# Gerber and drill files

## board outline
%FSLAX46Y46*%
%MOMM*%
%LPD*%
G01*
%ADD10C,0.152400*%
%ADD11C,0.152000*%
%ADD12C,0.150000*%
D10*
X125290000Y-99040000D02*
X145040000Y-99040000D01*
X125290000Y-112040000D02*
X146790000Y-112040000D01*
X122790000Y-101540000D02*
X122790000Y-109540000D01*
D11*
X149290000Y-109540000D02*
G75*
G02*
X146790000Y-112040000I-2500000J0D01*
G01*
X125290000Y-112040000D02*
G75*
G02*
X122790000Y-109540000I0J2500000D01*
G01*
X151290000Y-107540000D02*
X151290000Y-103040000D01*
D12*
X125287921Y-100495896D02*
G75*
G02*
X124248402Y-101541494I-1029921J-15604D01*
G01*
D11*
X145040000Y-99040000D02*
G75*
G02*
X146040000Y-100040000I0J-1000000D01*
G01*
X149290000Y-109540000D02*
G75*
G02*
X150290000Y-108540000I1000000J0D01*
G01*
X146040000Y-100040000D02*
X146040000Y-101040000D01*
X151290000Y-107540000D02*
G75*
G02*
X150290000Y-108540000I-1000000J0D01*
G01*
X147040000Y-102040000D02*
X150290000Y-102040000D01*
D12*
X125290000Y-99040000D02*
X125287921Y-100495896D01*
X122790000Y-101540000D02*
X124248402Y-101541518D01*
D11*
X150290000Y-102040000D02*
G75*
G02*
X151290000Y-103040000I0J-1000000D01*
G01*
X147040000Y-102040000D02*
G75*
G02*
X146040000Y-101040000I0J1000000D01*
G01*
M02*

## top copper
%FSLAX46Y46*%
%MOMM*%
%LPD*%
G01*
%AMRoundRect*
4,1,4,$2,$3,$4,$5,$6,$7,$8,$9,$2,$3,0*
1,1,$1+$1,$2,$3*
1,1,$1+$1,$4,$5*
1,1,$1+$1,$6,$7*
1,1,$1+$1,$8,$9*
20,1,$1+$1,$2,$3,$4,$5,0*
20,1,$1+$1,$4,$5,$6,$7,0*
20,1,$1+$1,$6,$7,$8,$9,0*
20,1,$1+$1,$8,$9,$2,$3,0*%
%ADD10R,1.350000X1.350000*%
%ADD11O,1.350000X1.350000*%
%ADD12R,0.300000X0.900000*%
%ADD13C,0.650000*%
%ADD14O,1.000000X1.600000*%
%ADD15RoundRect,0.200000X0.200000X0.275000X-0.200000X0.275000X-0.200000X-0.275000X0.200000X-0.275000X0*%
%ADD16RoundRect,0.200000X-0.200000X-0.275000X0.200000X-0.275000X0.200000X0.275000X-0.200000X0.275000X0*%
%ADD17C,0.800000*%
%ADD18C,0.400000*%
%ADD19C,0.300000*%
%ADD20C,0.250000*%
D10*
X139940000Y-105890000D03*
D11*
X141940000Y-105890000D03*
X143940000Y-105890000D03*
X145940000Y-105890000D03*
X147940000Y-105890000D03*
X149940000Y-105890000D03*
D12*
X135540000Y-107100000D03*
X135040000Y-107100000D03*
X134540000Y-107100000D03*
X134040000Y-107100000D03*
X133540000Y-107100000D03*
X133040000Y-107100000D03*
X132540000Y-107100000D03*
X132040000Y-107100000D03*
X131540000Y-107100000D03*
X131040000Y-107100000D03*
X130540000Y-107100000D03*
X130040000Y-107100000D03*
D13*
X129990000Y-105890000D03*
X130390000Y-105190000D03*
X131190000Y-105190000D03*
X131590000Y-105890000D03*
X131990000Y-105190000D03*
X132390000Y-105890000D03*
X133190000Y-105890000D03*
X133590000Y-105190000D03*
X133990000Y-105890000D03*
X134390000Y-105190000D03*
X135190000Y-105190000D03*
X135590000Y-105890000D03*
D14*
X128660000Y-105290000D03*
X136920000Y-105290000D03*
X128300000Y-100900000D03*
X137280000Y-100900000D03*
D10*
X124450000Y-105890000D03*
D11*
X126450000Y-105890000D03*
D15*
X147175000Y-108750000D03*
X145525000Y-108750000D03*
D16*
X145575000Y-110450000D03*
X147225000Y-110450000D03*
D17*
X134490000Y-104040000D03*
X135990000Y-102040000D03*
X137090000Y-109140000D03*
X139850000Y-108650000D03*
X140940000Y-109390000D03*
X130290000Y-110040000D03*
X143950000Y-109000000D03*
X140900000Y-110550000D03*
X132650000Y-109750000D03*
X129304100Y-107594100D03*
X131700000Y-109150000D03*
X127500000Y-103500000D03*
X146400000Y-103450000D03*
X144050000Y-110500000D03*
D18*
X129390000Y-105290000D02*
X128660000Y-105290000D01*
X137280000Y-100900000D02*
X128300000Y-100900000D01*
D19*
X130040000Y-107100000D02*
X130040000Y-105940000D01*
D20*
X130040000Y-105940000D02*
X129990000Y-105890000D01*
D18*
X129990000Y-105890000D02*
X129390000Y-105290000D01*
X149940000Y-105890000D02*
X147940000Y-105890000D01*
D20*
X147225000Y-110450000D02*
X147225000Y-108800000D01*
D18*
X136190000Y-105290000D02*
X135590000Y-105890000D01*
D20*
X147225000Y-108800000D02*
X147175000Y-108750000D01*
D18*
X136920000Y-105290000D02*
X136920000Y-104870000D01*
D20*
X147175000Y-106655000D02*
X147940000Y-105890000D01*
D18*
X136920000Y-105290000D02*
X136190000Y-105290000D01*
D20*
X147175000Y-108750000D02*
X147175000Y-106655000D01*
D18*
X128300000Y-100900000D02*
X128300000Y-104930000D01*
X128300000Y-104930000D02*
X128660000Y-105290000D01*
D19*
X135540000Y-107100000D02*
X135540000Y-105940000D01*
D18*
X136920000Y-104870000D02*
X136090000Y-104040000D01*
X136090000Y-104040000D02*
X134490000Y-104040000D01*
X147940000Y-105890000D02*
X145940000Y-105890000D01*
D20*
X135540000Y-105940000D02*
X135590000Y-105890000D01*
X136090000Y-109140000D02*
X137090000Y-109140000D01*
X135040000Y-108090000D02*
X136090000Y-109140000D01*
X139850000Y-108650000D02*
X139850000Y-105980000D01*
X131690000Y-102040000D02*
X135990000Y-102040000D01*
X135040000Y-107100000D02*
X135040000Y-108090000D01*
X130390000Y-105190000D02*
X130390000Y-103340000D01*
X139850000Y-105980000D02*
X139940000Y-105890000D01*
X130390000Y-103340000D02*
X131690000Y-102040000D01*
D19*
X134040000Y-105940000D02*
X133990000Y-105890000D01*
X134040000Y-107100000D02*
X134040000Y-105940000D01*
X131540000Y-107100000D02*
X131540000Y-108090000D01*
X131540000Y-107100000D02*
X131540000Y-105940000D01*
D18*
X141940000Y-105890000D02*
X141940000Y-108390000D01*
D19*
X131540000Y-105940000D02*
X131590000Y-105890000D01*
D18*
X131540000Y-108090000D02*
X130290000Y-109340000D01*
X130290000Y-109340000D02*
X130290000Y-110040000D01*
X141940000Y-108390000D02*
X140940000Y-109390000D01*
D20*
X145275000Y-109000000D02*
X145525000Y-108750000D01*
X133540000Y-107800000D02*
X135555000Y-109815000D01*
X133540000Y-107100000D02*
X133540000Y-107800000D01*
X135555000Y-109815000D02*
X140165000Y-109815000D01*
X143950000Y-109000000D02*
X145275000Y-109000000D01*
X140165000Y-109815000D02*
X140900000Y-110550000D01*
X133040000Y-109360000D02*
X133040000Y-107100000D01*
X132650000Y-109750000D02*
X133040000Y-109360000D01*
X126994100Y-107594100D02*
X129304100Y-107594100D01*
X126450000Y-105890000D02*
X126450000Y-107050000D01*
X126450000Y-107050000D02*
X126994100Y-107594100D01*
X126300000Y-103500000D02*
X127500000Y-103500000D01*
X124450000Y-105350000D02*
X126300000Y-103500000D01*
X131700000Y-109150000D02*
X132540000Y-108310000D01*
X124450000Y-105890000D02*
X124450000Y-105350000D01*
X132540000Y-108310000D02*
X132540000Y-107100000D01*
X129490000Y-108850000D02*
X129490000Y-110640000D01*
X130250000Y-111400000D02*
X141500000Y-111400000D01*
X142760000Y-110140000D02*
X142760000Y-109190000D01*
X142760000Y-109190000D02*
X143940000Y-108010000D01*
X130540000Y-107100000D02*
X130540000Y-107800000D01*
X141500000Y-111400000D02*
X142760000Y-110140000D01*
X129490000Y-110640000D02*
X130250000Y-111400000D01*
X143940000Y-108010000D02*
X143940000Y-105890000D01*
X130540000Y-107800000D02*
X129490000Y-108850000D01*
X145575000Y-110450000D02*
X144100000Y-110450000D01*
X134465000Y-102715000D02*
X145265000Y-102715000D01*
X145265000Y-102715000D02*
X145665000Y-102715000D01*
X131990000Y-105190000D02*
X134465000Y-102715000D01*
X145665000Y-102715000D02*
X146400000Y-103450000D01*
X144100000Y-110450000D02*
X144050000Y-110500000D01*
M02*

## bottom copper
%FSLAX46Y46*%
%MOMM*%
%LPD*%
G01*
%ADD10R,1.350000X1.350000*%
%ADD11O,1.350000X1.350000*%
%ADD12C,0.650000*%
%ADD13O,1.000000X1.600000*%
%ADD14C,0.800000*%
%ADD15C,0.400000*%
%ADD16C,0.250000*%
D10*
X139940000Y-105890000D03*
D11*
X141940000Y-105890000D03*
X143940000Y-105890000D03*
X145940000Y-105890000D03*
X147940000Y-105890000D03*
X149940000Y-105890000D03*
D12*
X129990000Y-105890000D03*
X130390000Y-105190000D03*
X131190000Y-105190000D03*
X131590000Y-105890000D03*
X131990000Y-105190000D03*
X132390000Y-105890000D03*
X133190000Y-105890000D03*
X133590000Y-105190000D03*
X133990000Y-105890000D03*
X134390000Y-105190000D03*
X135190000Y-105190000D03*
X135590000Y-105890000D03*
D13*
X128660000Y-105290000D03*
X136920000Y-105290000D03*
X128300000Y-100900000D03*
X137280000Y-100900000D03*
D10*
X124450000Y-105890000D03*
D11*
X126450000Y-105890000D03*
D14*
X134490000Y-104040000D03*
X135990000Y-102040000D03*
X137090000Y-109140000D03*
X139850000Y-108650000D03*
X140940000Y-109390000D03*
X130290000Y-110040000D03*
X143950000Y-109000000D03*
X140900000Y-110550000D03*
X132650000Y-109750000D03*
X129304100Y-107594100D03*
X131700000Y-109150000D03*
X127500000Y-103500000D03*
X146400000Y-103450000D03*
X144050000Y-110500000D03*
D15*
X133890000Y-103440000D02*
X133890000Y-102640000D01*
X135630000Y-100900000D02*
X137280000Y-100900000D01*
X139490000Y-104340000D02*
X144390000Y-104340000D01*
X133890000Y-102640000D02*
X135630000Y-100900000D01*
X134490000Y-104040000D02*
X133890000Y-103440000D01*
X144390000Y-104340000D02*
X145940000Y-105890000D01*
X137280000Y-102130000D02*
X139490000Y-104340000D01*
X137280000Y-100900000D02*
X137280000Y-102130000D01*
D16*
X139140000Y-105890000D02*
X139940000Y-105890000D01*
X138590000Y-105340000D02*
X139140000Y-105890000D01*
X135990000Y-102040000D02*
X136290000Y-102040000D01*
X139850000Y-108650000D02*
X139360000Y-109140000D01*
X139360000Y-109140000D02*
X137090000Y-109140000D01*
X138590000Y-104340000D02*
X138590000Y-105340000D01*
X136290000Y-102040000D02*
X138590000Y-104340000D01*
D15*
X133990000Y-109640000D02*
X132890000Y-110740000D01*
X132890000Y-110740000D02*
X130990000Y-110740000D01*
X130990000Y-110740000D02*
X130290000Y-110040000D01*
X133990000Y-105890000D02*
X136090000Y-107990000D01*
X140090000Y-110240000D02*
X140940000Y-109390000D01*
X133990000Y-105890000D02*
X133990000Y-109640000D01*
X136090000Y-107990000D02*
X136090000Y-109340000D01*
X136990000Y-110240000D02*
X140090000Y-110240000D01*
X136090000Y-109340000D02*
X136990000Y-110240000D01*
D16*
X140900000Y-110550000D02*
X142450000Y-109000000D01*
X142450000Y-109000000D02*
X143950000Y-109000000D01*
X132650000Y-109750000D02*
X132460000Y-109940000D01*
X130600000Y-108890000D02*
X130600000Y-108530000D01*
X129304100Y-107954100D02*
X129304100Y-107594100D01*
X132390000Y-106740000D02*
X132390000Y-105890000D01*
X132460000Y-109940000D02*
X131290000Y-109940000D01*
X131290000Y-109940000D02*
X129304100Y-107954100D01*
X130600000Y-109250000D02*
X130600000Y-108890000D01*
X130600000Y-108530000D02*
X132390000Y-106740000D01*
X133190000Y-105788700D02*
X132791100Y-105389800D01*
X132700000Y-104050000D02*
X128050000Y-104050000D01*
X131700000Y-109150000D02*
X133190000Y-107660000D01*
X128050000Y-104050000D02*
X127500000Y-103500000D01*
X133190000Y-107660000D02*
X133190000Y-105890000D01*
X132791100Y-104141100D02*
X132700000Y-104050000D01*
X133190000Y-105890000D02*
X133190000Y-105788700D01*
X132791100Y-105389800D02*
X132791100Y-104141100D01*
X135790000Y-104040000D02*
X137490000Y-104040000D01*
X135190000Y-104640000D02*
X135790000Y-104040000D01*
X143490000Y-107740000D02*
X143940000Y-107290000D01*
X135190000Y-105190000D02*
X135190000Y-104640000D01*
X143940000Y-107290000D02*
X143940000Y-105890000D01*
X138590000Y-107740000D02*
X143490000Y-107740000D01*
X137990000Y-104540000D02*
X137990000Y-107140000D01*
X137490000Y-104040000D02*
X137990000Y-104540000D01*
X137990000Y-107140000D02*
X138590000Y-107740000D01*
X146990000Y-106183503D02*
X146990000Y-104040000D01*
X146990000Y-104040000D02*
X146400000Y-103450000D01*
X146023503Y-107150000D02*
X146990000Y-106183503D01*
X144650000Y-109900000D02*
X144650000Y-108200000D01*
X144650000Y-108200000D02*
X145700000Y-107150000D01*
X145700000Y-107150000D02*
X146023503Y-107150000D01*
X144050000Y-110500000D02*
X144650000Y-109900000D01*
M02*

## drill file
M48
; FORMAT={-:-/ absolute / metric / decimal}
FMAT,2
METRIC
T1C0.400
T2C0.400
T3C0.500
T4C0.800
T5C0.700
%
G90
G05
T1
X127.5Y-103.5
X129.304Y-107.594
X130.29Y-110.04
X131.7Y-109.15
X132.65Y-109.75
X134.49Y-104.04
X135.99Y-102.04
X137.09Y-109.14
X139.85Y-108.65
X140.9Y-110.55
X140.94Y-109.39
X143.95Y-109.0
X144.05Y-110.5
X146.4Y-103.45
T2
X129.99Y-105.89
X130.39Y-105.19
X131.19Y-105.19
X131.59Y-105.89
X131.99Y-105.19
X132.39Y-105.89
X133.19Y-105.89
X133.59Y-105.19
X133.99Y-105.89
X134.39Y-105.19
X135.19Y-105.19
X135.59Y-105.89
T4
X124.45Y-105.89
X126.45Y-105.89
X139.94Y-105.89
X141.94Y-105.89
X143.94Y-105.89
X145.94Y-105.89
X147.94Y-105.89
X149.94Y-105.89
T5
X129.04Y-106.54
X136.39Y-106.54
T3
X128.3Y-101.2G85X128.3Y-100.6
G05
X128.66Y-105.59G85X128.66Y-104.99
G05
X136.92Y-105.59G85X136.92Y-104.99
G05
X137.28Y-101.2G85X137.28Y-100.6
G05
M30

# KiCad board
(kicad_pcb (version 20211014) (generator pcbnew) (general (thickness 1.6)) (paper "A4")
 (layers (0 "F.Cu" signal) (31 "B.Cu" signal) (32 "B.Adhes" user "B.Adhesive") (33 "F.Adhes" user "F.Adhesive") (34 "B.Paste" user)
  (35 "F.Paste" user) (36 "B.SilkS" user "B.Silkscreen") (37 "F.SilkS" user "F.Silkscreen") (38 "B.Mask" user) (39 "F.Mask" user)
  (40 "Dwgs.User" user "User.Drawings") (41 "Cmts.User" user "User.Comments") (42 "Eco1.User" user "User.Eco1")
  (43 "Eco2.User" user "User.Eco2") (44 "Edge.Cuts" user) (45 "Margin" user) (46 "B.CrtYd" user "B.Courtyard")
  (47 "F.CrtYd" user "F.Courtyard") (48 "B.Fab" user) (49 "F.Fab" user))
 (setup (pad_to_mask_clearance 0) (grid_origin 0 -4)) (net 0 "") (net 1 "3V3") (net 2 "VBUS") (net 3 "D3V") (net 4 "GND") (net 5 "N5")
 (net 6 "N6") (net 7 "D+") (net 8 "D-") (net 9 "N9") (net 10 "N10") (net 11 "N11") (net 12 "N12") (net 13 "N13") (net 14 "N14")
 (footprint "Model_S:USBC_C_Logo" (layer "F.Cu") (at 130.3 110)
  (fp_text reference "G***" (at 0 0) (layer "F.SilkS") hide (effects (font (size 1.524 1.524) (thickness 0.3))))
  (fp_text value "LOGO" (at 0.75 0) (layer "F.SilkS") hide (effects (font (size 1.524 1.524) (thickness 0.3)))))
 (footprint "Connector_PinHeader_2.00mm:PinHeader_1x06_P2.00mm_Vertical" (layer "F.Cu") (at 139.94 105.89 90)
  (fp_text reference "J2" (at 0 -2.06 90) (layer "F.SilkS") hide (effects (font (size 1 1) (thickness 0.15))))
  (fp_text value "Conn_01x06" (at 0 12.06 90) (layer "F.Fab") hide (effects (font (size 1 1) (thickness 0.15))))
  (pad "1" thru_hole rect locked (at 0 0 90) (size 1.35 1.35) (drill 0.8) (layers *.Cu *.Mask) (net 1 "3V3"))
  (pad "2" thru_hole oval locked (at 0 2 90) (size 1.35 1.35) (drill 0.8) (layers *.Cu *.Mask) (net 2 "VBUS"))
  (pad "3" thru_hole oval locked (at 0 4 90) (size 1.35 1.35) (drill 0.8) (layers *.Cu *.Mask) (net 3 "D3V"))
  (pad "4" thru_hole oval locked (at 0 6 90) (size 1.35 1.35) (drill 0.8) (layers *.Cu *.Mask) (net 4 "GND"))
  (pad "5" thru_hole oval locked (at 0 8 90) (size 1.35 1.35) (drill 0.8) (layers *.Cu *.Mask) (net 4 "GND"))
  (pad "6" thru_hole oval locked (at 0 10 90) (size 1.35 1.35) (drill 0.8) (layers *.Cu *.Mask) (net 4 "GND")))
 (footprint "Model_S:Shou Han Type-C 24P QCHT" (layer "F.Cu") (at 132.79 99.04 180)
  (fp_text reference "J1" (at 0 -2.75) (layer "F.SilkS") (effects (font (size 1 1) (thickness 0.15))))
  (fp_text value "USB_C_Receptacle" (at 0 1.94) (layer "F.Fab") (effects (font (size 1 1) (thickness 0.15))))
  (pad "" np_thru_hole circle locked (at 3.75 -7.5 180) (size 0.7 0.7) (drill 0.7) (layers *.Cu *.Mask))
  (pad "" np_thru_hole circle locked (at -3.6 -7.5 180) (size 0.7 0.7) (drill 0.7) (layers *.Cu *.Mask))
  (pad "A1" smd rect locked (at -2.75 -8.06 180) (size 0.3 0.9) (layers "F.Cu" "F.Paste" "F.Mask") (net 4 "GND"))
  (pad "A2" smd rect locked (at -2.25 -8.06 180) (size 0.3 0.9) (layers "F.Cu" "F.Paste" "F.Mask") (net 1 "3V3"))
  (pad "A3" smd rect locked (at -1.75 -8.06 180) (size 0.3 0.9) (layers "F.Cu" "F.Paste" "F.Mask") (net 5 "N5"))
  (pad "A4" smd rect locked (at -1.25 -8.06 180) (size 0.3 0.9) (layers "F.Cu" "F.Paste" "F.Mask") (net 2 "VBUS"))
  (pad "A5" smd rect locked (at -0.75 -8.06 180) (size 0.3 0.9) (layers "F.Cu" "F.Paste" "F.Mask") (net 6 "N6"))
  (pad "A6" smd rect locked (at -0.25 -8.06 180) (size 0.3 0.9) (layers "F.Cu" "F.Paste" "F.Mask") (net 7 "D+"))
  (pad "A7" smd rect locked (at 0.25 -8.06 180) (size 0.3 0.9) (layers "F.Cu" "F.Paste" "F.Mask") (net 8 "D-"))
  (pad "A8" smd rect locked (at 0.75 -8.06 180) (size 0.3 0.9) (layers "F.Cu" "F.Paste" "F.Mask") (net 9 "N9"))
  (pad "A9" smd rect locked (at 1.25 -8.06 180) (size 0.3 0.9) (layers "F.Cu" "F.Paste" "F.Mask") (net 2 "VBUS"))
  (pad "A10" smd rect locked (at 1.75 -8.06 180) (size 0.3 0.9) (layers "F.Cu" "F.Paste" "F.Mask") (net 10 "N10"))
  (pad "A11" smd rect locked (at 2.25 -8.06 180) (size 0.3 0.9) (layers "F.Cu" "F.Paste" "F.Mask") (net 3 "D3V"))
  (pad "A12" smd rect locked (at 2.75 -8.06 180) (size 0.3 0.9) (layers "F.Cu" "F.Paste" "F.Mask") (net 4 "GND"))
  (pad "B1" thru_hole circle locked (at 2.8 -6.85 180) (size 0.65 0.65) (drill 0.4) (layers *.Cu *.Mask) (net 4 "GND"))
  (pad "B2" thru_hole circle locked (at 2.4 -6.15 180) (size 0.65 0.65) (drill 0.4) (layers *.Cu *.Mask) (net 1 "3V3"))
  (pad "B3" thru_hole circle locked (at 1.6 -6.15 180) (size 0.65 0.65) (drill 0.4) (layers *.Cu *.Mask) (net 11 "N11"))
  (pad "B4" thru_hole circle locked (at 1.2 -6.85 180) (size 0.65 0.65) (drill 0.4) (layers *.Cu *.Mask) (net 2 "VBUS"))
  (pad "B5" thru_hole circle locked (at 0.8 -6.15 180) (size 0.65 0.65) (drill 0.4) (layers *.Cu *.Mask) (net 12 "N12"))
  (pad "B6" thru_hole circle locked (at 0.4 -6.85 180) (size 0.65 0.65) (drill 0.4) (layers *.Cu *.Mask) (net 7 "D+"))
  (pad "B7" thru_hole circle locked (at -0.4 -6.85 180) (size 0.65 0.65) (drill 0.4) (layers *.Cu *.Mask) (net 8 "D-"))
  (pad "B8" thru_hole circle locked (at -0.8 -6.15 180) (size 0.65 0.65) (drill 0.4) (layers *.Cu *.Mask) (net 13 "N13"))
  (pad "B9" thru_hole circle locked (at -1.2 -6.85 180) (size 0.65 0.65) (drill 0.4) (layers *.Cu *.Mask) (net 2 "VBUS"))
  (pad "B10" thru_hole circle locked (at -1.6 -6.15 180) (size 0.65 0.65) (drill 0.4) (layers *.Cu *.Mask) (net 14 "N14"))
  (pad "B11" thru_hole circle locked (at -2.4 -6.15 180) (size 0.65 0.65) (drill 0.4) (layers *.Cu *.Mask) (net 3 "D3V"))
  (pad "B12" thru_hole circle locked (at -2.8 -6.85 180) (size 0.65 0.65) (drill 0.4) (layers *.Cu *.Mask) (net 4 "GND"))
  (pad "S1" thru_hole oval locked (at 4.13 -6.25 180) (size 1 1.6) (drill oval 0.5 1.1) (layers *.Cu *.Mask) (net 4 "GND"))
  (pad "S1" thru_hole oval locked (at -4.13 -6.25 180) (size 1 1.6) (drill oval 0.5 1.1) (layers *.Cu *.Mask) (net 4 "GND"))
  (pad "S1" thru_hole oval locked (at 4.49 -1.86 180) (size 1 1.6) (drill oval 0.5 1.1) (layers *.Cu *.Mask) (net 4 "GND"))
  (pad "S1" thru_hole oval locked (at -4.49 -1.86 180) (size 1 1.6) (drill oval 0.5 1.1) (layers *.Cu *.Mask) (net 4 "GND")))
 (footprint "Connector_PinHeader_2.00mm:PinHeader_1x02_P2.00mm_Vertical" (layer "F.Cu") (at 124.45 105.89 90)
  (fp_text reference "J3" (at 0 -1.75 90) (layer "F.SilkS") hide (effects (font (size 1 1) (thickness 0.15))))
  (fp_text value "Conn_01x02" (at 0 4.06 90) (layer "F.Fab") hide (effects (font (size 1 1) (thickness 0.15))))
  (pad "1" thru_hole rect locked (at 0 0 90) (size 1.35 1.35) (drill 0.8) (layers *.Cu *.Mask) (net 8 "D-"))
  (pad "2" thru_hole oval locked (at 0 2 90) (size 1.35 1.35) (drill 0.8) (layers *.Cu *.Mask) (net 7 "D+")))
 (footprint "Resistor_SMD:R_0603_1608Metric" (layer "F.Cu") (at 146.35 108.75 180)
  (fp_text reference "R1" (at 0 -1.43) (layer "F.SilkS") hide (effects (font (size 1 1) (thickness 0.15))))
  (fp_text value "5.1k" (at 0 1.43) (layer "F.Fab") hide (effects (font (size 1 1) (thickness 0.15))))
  (pad "1" smd roundrect locked (at -0.825 0 180) (size 0.8 0.95) (layers "F.Cu" "F.Paste" "F.Mask") (roundrect_rratio 0.25) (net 4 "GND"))
  (pad "2" smd roundrect locked (at 0.825 0 180) (size 0.8 0.95) (layers "F.Cu" "F.Paste" "F.Mask") (roundrect_rratio 0.25) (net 6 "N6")))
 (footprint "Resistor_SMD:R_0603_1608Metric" (layer "F.Cu") (at 146.4 110.45)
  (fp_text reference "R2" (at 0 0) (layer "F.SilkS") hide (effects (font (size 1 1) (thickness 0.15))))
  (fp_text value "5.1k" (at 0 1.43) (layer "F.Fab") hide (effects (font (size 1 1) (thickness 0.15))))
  (pad "1" smd roundrect locked (at -0.825 0) (size 0.8 0.95) (layers "F.Cu" "F.Paste" "F.Mask") (roundrect_rratio 0.25) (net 12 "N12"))
  (pad "2" smd roundrect locked (at 0.825 0) (size 0.8 0.95) (layers "F.Cu" "F.Paste" "F.Mask") (roundrect_rratio 0.25) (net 4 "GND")))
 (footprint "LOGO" (layer "F.Cu") (at 125.453205 109.842378)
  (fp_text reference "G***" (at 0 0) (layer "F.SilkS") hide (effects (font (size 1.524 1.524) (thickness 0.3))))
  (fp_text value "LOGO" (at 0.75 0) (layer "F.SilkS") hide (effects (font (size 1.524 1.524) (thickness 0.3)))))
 (gr_line (start 125.29 99.04) (end 145.04 99.04) (layer "Edge.Cuts") (width 0.1524))
 (gr_line (start 125.29 112.04) (end 146.79 112.04) (layer "Edge.Cuts") (width 0.1524))
 (gr_line (start 122.79 101.54) (end 122.79 109.54) (layer "Edge.Cuts") (width 0.1524))
 (gr_arc (start 149.29 109.54) (mid 148.557767 111.307767) (end 146.79 112.04) (layer "Edge.Cuts") (width 0.152))
 (gr_arc (start 125.29 112.04) (mid 123.522233 111.307767) (end 122.79 109.54) (layer "Edge.Cuts") (width 0.152))
 (gr_line (start 151.29 107.54) (end 151.29 103.04) (layer "Edge.Cuts") (width 0.152))
 (gr_arc (start 125.287921 100.495896) (mid 124.988467 101.237726) (end 124.248402 101.541518) (layer "Edge.Cuts") (width 0.15))
 (gr_arc (start 145.04 99.04) (mid 145.747107 99.332893) (end 146.04 100.04) (layer "Edge.Cuts") (width 0.152))
 (gr_arc (start 149.29 109.54) (mid 149.582893 108.832893) (end 150.29 108.54) (layer "Edge.Cuts") (width 0.152))
 (gr_line (start 146.04 100.04) (end 146.04 101.04) (layer "Edge.Cuts") (width 0.152))
 (gr_arc (start 151.29 107.54) (mid 150.997107 108.247107) (end 150.29 108.54) (layer "Edge.Cuts") (width 0.152))
 (gr_line (start 147.04 102.04) (end 150.29 102.04) (layer "Edge.Cuts") (width 0.152))
 (gr_line (start 125.29 99.04) (end 125.287921 100.495896) (layer "Edge.Cuts") (width 0.15))
 (gr_line (start 122.79 101.54) (end 124.248402 101.541518) (layer "Edge.Cuts") (width 0.15))
 (gr_arc (start 150.29 102.04) (mid 150.997107 102.332893) (end 151.29 103.04) (layer "Edge.Cuts") (width 0.152))
 (gr_arc (start 147.04 102.04) (mid 146.332893 101.747107) (end 146.04 101.04) (layer "Edge.Cuts") (width 0.152))
 (segment (start 129.39 105.29) (end 128.66 105.29) (width 0.4) (layer "F.Cu") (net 4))
 (segment (start 137.28 100.9) (end 128.3 100.9) (width 0.4) (layer "F.Cu") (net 4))
 (segment (start 130.04 107.1) (end 130.04 105.94) (width 0.3) (layer "F.Cu") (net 4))
 (segment (start 130.04 105.94) (end 129.99 105.89) (width 0.25) (layer "F.Cu") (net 4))
 (segment (start 129.99 105.89) (end 129.39 105.29) (width 0.4) (layer "F.Cu") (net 4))
 (segment (start 149.94 105.89) (end 147.94 105.89) (width 0.4) (layer "F.Cu") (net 4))
 (segment (start 147.225 110.45) (end 147.225 108.8) (width 0.25) (layer "F.Cu") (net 4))
 (segment (start 136.19 105.29) (end 135.59 105.89) (width 0.4) (layer "F.Cu") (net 4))
 (segment (start 147.225 108.8) (end 147.175 108.75) (width 0.25) (layer "F.Cu") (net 4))
 (segment (start 136.92 105.29) (end 136.92 104.87) (width 0.4) (layer "F.Cu") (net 4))
 (segment (start 147.175 106.655) (end 147.94 105.89) (width 0.25) (layer "F.Cu") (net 4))
 (segment (start 136.92 105.29) (end 136.19 105.29) (width 0.4) (layer "F.Cu") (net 4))
 (segment (start 147.175 108.75) (end 147.175 106.655) (width 0.25) (layer "F.Cu") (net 4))
 (segment (start 128.3 100.9) (end 128.3 104.93) (width 0.4) (layer "F.Cu") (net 4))
 (segment (start 128.3 104.93) (end 128.66 105.29) (width 0.4) (layer "F.Cu") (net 4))
 (segment (start 135.54 107.1) (end 135.54 105.94) (width 0.3) (layer "F.Cu") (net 4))
 (segment (start 136.92 104.87) (end 136.09 104.04) (width 0.4) (layer "F.Cu") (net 4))
 (segment (start 136.09 104.04) (end 134.49 104.04) (width 0.4) (layer "F.Cu") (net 4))
 (segment (start 147.94 105.89) (end 145.94 105.89) (width 0.4) (layer "F.Cu") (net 4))
 (segment (start 135.54 105.94) (end 135.59 105.89) (width 0.25) (layer "F.Cu") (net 4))
 (via (at 134.49 104.04) (size 0.8) (drill 0.4) (layers "F.Cu" "B.Cu") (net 4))
 (segment (start 133.89 103.44) (end 133.89 102.64) (width 0.4) (layer "B.Cu") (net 4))
 (segment (start 135.63 100.9) (end 137.28 100.9) (width 0.4) (layer "B.Cu") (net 4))
 (segment (start 139.49 104.34) (end 144.39 104.34) (width 0.4) (layer "B.Cu") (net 4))
 (segment (start 133.89 102.64) (end 135.63 100.9) (width 0.4) (layer "B.Cu") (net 4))
 (segment (start 134.49 104.04) (end 133.89 103.44) (width 0.4) (layer "B.Cu") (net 4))
 (segment (start 144.39 104.34) (end 145.94 105.89) (width 0.4) (layer "B.Cu") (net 4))
 (segment (start 137.28 102.13) (end 139.49 104.34) (width 0.4) (layer "B.Cu") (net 4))
 (segment (start 137.28 100.9) (end 137.28 102.13) (width 0.4) (layer "B.Cu") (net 4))
 (segment (start 136.09 109.14) (end 137.09 109.14) (width 0.25) (layer "F.Cu") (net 1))
 (segment (start 135.04 108.09) (end 136.09 109.14) (width 0.25) (layer "F.Cu") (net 1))
 (segment (start 139.85 108.65) (end 139.85 105.98) (width 0.25) (layer "F.Cu") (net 1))
 (segment (start 131.69 102.04) (end 135.99 102.04) (width 0.25) (layer "F.Cu") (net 1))
 (segment (start 135.04 107.1) (end 135.04 108.09) (width 0.25) (layer "F.Cu") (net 1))
 (segment (start 130.39 105.19) (end 130.39 103.34) (width 0.25) (layer "F.Cu") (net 1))
 (segment (start 139.85 105.98) (end 139.94 105.89) (width 0.25) (layer "F.Cu") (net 1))
 (segment (start 130.39 103.34) (end 131.69 102.04) (width 0.25) (layer "F.Cu") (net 1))
 (via (at 135.99 102.04) (size 0.8) (drill 0.4) (layers "F.Cu" "B.Cu") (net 1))
 (via (at 137.09 109.14) (size 0.8) (drill 0.4) (layers "F.Cu" "B.Cu") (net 1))
 (via (at 139.85 108.65) (size 0.8) (drill 0.4) (layers "F.Cu" "B.Cu") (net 1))
 (segment (start 139.14 105.89) (end 139.94 105.89) (width 0.25) (layer "B.Cu") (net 1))
 (segment (start 138.59 105.34) (end 139.14 105.89) (width 0.25) (layer "B.Cu") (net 1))
 (segment (start 135.99 102.04) (end 136.29 102.04) (width 0.25) (layer "B.Cu") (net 1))
 (segment (start 139.85 108.65) (end 139.36 109.14) (width 0.25) (layer "B.Cu") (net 1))
 (segment (start 139.36 109.14) (end 137.09 109.14) (width 0.25) (layer "B.Cu") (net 1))
 (segment (start 138.59 104.34) (end 138.59 105.34) (width 0.25) (layer "B.Cu") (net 1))
 (segment (start 136.29 102.04) (end 138.59 104.34) (width 0.25) (layer "B.Cu") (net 1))
 (segment (start 134.04 105.94) (end 133.99 105.89) (width 0.3) (layer "F.Cu") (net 2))
 (segment (start 134.04 107.1) (end 134.04 105.94) (width 0.3) (layer "F.Cu") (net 2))
 (segment (start 131.54 107.1) (end 131.54 108.09) (width 0.3) (layer "F.Cu") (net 2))
 (segment (start 131.54 107.1) (end 131.54 105.94) (width 0.3) (layer "F.Cu") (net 2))
 (segment (start 141.94 105.89) (end 141.94 108.39) (width 0.4) (layer "F.Cu") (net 2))
 (segment (start 131.54 105.94) (end 131.59 105.89) (width 0.3) (layer "F.Cu") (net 2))
 (segment (start 131.54 108.09) (end 130.29 109.34) (width 0.4) (layer "F.Cu") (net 2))
 (segment (start 130.29 109.34) (end 130.29 110.04) (width 0.4) (layer "F.Cu") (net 2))
 (segment (start 141.94 108.39) (end 140.94 109.39) (width 0.4) (layer "F.Cu") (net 2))
 (via (at 140.94 109.39) (size 0.8) (drill 0.4) (layers "F.Cu" "B.Cu") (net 2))
 (via (at 130.29 110.04) (size 0.8) (drill 0.4) (layers "F.Cu" "B.Cu") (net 2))
 (segment (start 133.99 109.64) (end 132.89 110.74) (width 0.4) (layer "B.Cu") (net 2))
 (segment (start 132.89 110.74) (end 130.99 110.74) (width 0.4) (layer "B.Cu") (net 2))
 (segment (start 130.99 110.74) (end 130.29 110.04) (width 0.4) (layer "B.Cu") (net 2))
 (segment (start 133.99 105.89) (end 136.09 107.99) (width 0.4) (layer "B.Cu") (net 2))
 (segment (start 140.09 110.24) (end 140.94 109.39) (width 0.4) (layer "B.Cu") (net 2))
 (segment (start 133.99 105.89) (end 133.99 109.64) (width 0.4) (layer "B.Cu") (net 2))
 (segment (start 136.09 107.99) (end 136.09 109.34) (width 0.4) (layer "B.Cu") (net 2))
 (segment (start 136.99 110.24) (end 140.09 110.24) (width 0.4) (layer "B.Cu") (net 2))
 (segment (start 136.09 109.34) (end 136.99 110.24) (width 0.4) (layer "B.Cu") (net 2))
 (segment (start 145.275 109) (end 145.525 108.75) (width 0.25) (layer "F.Cu") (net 6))
 (segment (start 133.54 107.8) (end 135.555 109.815) (width 0.25) (layer "F.Cu") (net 6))
 (segment (start 133.54 107.1) (end 133.54 107.8) (width 0.25) (layer "F.Cu") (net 6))
 (segment (start 135.555 109.815) (end 140.165 109.815) (width 0.25) (layer "F.Cu") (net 6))
 (segment (start 143.95 109) (end 145.275 109) (width 0.25) (layer "F.Cu") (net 6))
 (segment (start 140.165 109.815) (end 140.9 110.55) (width 0.25) (layer "F.Cu") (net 6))
 (via (at 143.95 109) (size 0.8) (drill 0.4) (layers "F.Cu" "B.Cu") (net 6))
 (via (at 140.9 110.55) (size 0.8) (drill 0.4) (layers "F.Cu" "B.Cu") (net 6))
 (segment (start 140.9 110.55) (end 142.45 109) (width 0.25) (layer "B.Cu") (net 6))
 (segment (start 142.45 109) (end 143.95 109) (width 0.25) (layer "B.Cu") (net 6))
 (segment (start 133.04 109.36) (end 133.04 107.1) (width 0.25) (layer "F.Cu") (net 7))
 (segment (start 132.65 109.75) (end 133.04 109.36) (width 0.25) (layer "F.Cu") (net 7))
 (segment (start 126.9941 107.5941) (end 129.3041 107.5941) (width 0.25) (layer "F.Cu") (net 7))
 (segment (start 126.45 105.89) (end 126.45 107.05) (width 0.25) (layer "F.Cu") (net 7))
 (segment (start 126.45 107.05) (end 126.9941 107.5941) (width 0.25) (layer "F.Cu") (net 7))
 (via (at 132.65 109.75) (size 0.8) (drill 0.4) (layers "F.Cu" "B.Cu") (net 7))
 (via (at 129.3041 107.5941) (size 0.8) (drill 0.4) (layers "F.Cu" "B.Cu") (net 7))
 (segment (start 132.65 109.75) (end 132.46 109.94) (width 0.25) (layer "B.Cu") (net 7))
 (segment (start 130.6 108.89) (end 130.6 108.53) (width 0.25) (layer "B.Cu") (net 7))
 (segment (start 129.3041 107.9541) (end 129.3041 107.5941) (width 0.25) (layer "B.Cu") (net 7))
 (segment (start 132.39 106.74) (end 132.39 105.89) (width 0.25) (layer "B.Cu") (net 7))
 (segment (start 132.46 109.94) (end 131.29 109.94) (width 0.25) (layer "B.Cu") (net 7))
 (segment (start 131.29 109.94) (end 129.3041 107.9541) (width 0.25) (layer "B.Cu") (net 7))
 (segment (start 130.6 109.25) (end 130.6 108.89) (width 0.25) (layer "B.Cu") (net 7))
 (segment (start 130.6 108.53) (end 132.39 106.74) (width 0.25) (layer "B.Cu") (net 7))
 (segment (start 126.3 103.5) (end 127.5 103.5) (width 0.25) (layer "F.Cu") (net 8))
 (segment (start 124.45 105.35) (end 126.3 103.5) (width 0.25) (layer "F.Cu") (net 8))
 (segment (start 131.7 109.15) (end 132.54 108.31) (width 0.25) (layer "F.Cu") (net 8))
 (segment (start 124.45 105.89) (end 124.45 105.35) (width 0.25) (layer "F.Cu") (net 8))
 (segment (start 132.54 108.31) (end 132.54 107.1) (width 0.25) (layer "F.Cu") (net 8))
 (via (at 131.7 109.15) (size 0.8) (drill 0.4) (layers "F.Cu" "B.Cu") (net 8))
 (via (at 127.5 103.5) (size 0.8) (drill 0.4) (layers "F.Cu" "B.Cu") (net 8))
 (segment (start 133.19 105.7887) (end 132.7911 105.3898) (width 0.25) (layer "B.Cu") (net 8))
 (segment (start 132.7 104.05) (end 128.05 104.05) (width 0.25) (layer "B.Cu") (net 8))
 (segment (start 131.7 109.15) (end 133.19 107.66) (width 0.25) (layer "B.Cu") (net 8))
 (segment (start 128.05 104.05) (end 127.5 103.5) (width 0.25) (layer "B.Cu") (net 8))
 (segment (start 133.19 107.66) (end 133.19 105.89) (width 0.25) (layer "B.Cu") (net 8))
 (segment (start 132.7911 104.1411) (end 132.7 104.05) (width 0.25) (layer "B.Cu") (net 8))
 (segment (start 133.19 105.89) (end 133.19 105.7887) (width 0.25) (layer "B.Cu") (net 8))
 (segment (start 132.7911 105.3898) (end 132.7911 104.1411) (width 0.25) (layer "B.Cu") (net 8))
 (segment (start 129.49 108.85) (end 129.49 110.64) (width 0.25) (layer "F.Cu") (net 3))
 (segment (start 130.25 111.4) (end 141.5 111.4) (width 0.25) (layer "F.Cu") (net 3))
 (segment (start 142.76 110.14) (end 142.76 109.19) (width 0.25) (layer "F.Cu") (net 3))
 (segment (start 142.76 109.19) (end 143.94 108.01) (width 0.25) (layer "F.Cu") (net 3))
 (segment (start 130.54 107.1) (end 130.54 107.8) (width 0.25) (layer "F.Cu") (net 3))
 (segment (start 141.5 111.4) (end 142.76 110.14) (width 0.25) (layer "F.Cu") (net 3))
 (segment (start 129.49 110.64) (end 130.25 111.4) (width 0.25) (layer "F.Cu") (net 3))
 (segment (start 143.94 108.01) (end 143.94 105.89) (width 0.25) (layer "F.Cu") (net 3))
 (segment (start 130.54 107.8) (end 129.49 108.85) (width 0.25) (layer "F.Cu") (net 3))
 (segment (start 135.79 104.04) (end 137.49 104.04) (width 0.25) (layer "B.Cu") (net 3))
 (segment (start 135.19 104.64) (end 135.79 104.04) (width 0.25) (layer "B.Cu") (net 3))
 (segment (start 143.49 107.74) (end 143.94 107.29) (width 0.25) (layer "B.Cu") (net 3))
 (segment (start 135.19 105.19) (end 135.19 104.64) (width 0.25) (layer "B.Cu") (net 3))
 (segment (start 143.94 107.29) (end 143.94 105.89) (width 0.25) (layer "B.Cu") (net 3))
 (segment (start 138.59 107.74) (end 143.49 107.74) (width 0.25) (layer "B.Cu") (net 3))
 (segment (start 137.99 104.54) (end 137.99 107.14) (width 0.25) (layer "B.Cu") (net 3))
 (segment (start 137.49 104.04) (end 137.99 104.54) (width 0.25) (layer "B.Cu") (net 3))
 (segment (start 137.99 107.14) (end 138.59 107.74) (width 0.25) (layer "B.Cu") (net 3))
 (segment (start 145.575 110.45) (end 144.1 110.45) (width 0.25) (layer "F.Cu") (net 12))
 (segment (start 134.465 102.715) (end 145.265 102.715) (width 0.25) (layer "F.Cu") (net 12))
 (segment (start 145.265 102.715) (end 145.665 102.715) (width 0.25) (layer "F.Cu") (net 12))
 (segment (start 131.99 105.19) (end 134.465 102.715) (width 0.25) (layer "F.Cu") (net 12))
 (segment (start 145.665 102.715) (end 146.4 103.45) (width 0.25) (layer "F.Cu") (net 12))
 (segment (start 144.1 110.45) (end 144.05 110.5) (width 0.25) (layer "F.Cu") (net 12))
 (via (at 146.4 103.45) (size 0.8) (drill 0.4) (layers "F.Cu" "B.Cu") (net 12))
 (via (at 144.05 110.5) (size 0.8) (drill 0.4) (layers "F.Cu" "B.Cu") (free) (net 12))
 (segment (start 146.99 106.183503) (end 146.99 104.04) (width 0.25) (layer "B.Cu") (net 12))
 (segment (start 146.99 104.04) (end 146.4 103.45) (width 0.25) (layer "B.Cu") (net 12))
 (segment (start 146.023503 107.15) (end 146.99 106.183503) (width 0.25) (layer "B.Cu") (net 12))
 (segment (start 144.65 109.9) (end 144.65 108.2) (width 0.25) (layer "B.Cu") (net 12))
 (segment (start 144.65 108.2) (end 145.7 107.15) (width 0.25) (layer "B.Cu") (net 12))
 (segment (start 145.7 107.15) (end 146.023503 107.15) (width 0.25) (layer "B.Cu") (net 12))
 (segment (start 144.05 110.5) (end 144.65 109.9) (width 0.25) (layer "B.Cu") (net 12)))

